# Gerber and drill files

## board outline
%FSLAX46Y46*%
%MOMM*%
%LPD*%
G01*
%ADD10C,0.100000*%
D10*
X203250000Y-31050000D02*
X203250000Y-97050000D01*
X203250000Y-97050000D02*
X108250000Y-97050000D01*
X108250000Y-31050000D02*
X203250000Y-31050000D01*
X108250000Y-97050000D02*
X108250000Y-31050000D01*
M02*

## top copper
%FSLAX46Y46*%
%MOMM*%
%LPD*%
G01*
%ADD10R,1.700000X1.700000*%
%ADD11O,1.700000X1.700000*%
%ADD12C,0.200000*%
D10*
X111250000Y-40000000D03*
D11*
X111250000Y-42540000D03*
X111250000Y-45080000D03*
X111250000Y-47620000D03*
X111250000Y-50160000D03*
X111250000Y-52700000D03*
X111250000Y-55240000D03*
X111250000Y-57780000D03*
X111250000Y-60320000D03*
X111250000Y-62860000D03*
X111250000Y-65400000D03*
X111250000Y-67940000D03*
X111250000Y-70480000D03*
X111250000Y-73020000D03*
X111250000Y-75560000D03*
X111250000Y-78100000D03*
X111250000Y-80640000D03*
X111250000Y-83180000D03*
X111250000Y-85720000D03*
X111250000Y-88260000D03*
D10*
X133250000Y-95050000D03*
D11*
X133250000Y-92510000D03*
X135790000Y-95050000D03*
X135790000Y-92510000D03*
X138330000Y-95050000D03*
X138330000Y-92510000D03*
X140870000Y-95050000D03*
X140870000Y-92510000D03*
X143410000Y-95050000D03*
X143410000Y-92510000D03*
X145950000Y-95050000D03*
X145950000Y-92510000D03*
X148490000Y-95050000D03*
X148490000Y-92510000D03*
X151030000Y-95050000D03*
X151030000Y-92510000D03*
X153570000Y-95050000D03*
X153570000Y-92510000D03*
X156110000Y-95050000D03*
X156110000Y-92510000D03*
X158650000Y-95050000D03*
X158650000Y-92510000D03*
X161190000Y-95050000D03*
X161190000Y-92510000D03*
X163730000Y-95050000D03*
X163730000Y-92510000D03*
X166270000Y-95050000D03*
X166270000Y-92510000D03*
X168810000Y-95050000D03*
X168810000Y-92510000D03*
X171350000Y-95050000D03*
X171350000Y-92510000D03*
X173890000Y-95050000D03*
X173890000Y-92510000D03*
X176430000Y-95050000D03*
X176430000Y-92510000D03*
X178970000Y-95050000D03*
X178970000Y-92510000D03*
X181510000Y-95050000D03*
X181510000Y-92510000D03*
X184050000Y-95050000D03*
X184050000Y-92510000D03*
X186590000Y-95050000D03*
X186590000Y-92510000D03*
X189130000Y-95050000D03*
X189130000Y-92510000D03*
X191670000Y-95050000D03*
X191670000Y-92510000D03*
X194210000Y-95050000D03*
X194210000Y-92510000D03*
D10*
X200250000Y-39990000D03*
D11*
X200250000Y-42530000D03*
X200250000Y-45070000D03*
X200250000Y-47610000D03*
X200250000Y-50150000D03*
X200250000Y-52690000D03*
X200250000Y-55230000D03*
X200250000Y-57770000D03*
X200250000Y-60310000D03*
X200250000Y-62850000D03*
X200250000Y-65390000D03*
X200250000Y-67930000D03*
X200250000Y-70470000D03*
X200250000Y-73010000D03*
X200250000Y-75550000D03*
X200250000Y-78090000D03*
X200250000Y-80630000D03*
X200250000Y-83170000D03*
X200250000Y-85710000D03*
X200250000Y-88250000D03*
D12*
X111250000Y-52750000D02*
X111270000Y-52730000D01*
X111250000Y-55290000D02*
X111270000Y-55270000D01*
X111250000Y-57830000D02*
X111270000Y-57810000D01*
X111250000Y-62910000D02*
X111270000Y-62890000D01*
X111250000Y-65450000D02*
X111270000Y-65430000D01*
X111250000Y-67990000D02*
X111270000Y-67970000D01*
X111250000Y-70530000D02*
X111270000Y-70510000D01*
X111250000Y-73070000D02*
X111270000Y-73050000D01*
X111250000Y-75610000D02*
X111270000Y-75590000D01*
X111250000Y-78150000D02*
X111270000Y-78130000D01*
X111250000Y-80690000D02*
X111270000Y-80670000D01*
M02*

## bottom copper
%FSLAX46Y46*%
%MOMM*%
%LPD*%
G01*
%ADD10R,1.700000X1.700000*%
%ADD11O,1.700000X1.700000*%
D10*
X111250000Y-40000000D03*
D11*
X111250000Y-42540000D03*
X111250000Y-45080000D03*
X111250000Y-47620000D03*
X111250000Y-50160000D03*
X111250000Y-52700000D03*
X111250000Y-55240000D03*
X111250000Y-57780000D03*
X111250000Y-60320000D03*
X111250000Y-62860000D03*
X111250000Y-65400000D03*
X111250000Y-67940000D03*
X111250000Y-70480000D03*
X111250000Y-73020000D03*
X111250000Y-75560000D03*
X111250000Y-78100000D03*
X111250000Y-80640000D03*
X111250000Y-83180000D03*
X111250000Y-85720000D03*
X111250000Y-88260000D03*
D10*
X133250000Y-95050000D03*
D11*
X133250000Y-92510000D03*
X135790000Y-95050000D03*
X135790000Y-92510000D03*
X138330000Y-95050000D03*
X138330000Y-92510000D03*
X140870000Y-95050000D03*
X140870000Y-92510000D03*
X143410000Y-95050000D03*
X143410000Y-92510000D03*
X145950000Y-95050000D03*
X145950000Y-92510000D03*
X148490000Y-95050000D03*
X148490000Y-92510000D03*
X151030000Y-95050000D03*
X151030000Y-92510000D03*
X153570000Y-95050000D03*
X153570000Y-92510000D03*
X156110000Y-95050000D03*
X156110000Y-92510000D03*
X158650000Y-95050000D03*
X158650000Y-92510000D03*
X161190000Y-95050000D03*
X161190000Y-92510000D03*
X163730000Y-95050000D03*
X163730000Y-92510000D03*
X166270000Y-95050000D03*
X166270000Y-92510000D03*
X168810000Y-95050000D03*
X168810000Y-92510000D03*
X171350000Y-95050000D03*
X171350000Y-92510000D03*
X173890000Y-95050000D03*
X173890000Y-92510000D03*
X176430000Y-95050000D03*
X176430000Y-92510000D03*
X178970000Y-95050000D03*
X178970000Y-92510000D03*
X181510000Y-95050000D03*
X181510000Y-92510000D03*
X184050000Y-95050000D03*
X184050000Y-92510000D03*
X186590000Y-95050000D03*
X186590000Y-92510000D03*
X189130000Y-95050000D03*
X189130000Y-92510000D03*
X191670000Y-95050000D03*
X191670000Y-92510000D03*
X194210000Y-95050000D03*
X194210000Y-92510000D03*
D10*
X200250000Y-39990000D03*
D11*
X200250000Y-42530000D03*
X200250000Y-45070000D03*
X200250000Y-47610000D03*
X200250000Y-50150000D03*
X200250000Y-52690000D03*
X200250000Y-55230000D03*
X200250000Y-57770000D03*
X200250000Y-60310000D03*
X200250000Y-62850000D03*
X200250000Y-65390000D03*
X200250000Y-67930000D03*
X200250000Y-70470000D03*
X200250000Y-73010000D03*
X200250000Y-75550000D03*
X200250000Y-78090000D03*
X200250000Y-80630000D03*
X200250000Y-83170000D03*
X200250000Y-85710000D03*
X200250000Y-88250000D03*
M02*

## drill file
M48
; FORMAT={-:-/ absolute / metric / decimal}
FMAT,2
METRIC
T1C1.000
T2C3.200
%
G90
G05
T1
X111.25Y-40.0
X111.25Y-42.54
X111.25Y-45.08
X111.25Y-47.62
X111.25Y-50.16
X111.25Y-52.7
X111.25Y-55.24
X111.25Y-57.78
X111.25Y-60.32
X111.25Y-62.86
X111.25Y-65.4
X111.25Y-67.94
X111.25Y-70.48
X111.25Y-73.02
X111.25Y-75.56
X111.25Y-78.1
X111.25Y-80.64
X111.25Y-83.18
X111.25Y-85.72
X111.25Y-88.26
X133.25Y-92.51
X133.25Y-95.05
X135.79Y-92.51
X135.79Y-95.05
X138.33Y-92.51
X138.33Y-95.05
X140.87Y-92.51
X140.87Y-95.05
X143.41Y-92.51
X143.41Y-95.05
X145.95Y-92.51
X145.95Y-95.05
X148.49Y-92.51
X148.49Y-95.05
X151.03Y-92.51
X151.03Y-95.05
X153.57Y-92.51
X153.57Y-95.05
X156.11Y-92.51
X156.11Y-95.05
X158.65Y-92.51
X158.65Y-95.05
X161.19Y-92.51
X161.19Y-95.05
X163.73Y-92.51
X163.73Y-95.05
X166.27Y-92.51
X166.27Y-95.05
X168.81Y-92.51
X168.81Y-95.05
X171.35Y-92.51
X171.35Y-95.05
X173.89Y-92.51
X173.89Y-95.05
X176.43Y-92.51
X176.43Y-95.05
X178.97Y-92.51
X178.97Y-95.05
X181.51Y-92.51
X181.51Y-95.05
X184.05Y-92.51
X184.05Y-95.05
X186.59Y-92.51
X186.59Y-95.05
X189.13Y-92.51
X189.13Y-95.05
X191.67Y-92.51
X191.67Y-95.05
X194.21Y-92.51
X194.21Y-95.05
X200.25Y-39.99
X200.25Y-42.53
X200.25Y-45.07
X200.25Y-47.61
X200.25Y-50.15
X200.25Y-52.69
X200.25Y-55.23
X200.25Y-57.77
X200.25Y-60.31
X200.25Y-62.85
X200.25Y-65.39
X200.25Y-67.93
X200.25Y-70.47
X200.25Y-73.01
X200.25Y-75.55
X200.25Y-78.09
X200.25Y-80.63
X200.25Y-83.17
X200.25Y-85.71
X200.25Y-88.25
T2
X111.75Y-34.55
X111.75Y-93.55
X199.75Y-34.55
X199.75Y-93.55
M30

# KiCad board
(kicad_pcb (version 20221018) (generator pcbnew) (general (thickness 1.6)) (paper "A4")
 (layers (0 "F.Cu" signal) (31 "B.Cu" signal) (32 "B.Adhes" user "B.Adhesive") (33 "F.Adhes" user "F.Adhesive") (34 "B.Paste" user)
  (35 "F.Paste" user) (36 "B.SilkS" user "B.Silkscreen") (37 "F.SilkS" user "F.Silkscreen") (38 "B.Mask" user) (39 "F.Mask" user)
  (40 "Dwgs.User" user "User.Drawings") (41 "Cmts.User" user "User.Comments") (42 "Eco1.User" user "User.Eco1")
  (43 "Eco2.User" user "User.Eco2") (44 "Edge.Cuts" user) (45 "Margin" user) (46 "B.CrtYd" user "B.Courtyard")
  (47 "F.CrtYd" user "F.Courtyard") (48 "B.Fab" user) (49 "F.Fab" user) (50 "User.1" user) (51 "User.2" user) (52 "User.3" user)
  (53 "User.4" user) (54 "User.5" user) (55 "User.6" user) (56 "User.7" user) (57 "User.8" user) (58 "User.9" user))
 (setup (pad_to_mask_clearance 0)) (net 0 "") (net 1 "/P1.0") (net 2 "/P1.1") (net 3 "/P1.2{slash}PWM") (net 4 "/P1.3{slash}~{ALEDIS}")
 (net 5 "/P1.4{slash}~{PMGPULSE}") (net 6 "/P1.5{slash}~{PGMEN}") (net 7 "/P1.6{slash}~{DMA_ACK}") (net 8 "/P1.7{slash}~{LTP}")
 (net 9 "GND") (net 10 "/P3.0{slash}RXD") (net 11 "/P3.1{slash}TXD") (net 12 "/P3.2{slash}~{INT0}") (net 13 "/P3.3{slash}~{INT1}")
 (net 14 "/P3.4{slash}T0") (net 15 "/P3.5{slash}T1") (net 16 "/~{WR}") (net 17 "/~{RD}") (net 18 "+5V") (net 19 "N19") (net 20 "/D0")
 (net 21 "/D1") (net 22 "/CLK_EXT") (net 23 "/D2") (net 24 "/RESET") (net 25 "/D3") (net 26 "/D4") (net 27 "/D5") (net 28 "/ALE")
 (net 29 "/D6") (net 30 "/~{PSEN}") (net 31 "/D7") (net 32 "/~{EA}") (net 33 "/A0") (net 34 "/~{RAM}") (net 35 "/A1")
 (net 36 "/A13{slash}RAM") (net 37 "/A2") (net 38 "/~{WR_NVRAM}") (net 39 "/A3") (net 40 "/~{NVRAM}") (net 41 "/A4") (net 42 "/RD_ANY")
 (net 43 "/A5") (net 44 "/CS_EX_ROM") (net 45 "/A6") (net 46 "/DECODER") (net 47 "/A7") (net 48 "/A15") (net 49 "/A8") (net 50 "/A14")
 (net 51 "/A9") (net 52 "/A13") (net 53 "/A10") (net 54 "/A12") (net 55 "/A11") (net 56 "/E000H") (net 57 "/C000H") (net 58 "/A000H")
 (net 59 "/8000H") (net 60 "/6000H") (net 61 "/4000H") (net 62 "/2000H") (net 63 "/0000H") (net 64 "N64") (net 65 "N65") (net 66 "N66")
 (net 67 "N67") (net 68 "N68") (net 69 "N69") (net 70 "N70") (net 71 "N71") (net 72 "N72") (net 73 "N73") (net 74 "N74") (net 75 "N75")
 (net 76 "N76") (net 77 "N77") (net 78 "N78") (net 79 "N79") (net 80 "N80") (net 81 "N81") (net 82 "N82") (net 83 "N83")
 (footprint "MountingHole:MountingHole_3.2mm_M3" (layer "F.Cu") (at 199.75 93.55)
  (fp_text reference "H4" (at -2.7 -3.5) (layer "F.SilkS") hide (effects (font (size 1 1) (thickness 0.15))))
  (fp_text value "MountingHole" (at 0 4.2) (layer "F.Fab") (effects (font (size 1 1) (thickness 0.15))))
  (pad "" np_thru_hole circle (at 0 0) (size 3.2 3.2) (drill 3.2) (layers "F&B.Cu" "*.Mask")))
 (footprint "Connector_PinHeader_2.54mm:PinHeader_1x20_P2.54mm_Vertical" (layer "F.Cu") (at 111.25 40)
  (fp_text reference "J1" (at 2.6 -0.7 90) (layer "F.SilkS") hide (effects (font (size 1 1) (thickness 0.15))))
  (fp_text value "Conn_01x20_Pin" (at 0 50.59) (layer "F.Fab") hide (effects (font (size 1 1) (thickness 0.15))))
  (pad "1" thru_hole rect (at 0 0) (size 1.7 1.7) (drill 1) (layers "*.Cu" "*.Mask") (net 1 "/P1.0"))
  (pad "2" thru_hole oval (at 0 2.54) (size 1.7 1.7) (drill 1) (layers "*.Cu" "*.Mask") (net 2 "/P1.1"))
  (pad "3" thru_hole oval (at 0 5.08) (size 1.7 1.7) (drill 1) (layers "*.Cu" "*.Mask") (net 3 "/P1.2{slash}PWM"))
  (pad "4" thru_hole oval (at 0 7.62) (size 1.7 1.7) (drill 1) (layers "*.Cu" "*.Mask") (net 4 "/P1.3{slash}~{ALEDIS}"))
  (pad "5" thru_hole oval (at 0 10.16) (size 1.7 1.7) (drill 1) (layers "*.Cu" "*.Mask") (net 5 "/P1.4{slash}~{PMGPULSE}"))
  (pad "6" thru_hole oval (at 0 12.7) (size 1.7 1.7) (drill 1) (layers "*.Cu" "*.Mask") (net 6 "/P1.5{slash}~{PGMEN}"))
  (pad "7" thru_hole oval (at 0 15.24) (size 1.7 1.7) (drill 1) (layers "*.Cu" "*.Mask") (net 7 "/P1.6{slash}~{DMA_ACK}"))
  (pad "8" thru_hole oval (at 0 17.78) (size 1.7 1.7) (drill 1) (layers "*.Cu" "*.Mask") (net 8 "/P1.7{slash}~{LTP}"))
  (pad "9" thru_hole oval (at 0 20.32) (size 1.7 1.7) (drill 1) (layers "*.Cu" "*.Mask") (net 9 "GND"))
  (pad "10" thru_hole oval (at 0 22.86) (size 1.7 1.7) (drill 1) (layers "*.Cu" "*.Mask") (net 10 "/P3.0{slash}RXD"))
  (pad "11" thru_hole oval (at 0 25.4) (size 1.7 1.7) (drill 1) (layers "*.Cu" "*.Mask") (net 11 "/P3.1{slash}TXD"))
  (pad "12" thru_hole oval (at 0 27.94) (size 1.7 1.7) (drill 1) (layers "*.Cu" "*.Mask") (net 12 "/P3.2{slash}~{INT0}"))
  (pad "13" thru_hole oval (at 0 30.48) (size 1.7 1.7) (drill 1) (layers "*.Cu" "*.Mask") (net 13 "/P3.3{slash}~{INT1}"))
  (pad "14" thru_hole oval (at 0 33.02) (size 1.7 1.7) (drill 1) (layers "*.Cu" "*.Mask") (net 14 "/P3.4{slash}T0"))
  (pad "15" thru_hole oval (at 0 35.56) (size 1.7 1.7) (drill 1) (layers "*.Cu" "*.Mask") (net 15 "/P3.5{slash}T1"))
  (pad "16" thru_hole oval (at 0 38.1) (size 1.7 1.7) (drill 1) (layers "*.Cu" "*.Mask") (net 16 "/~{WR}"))
  (pad "17" thru_hole oval (at 0 40.64) (size 1.7 1.7) (drill 1) (layers "*.Cu" "*.Mask") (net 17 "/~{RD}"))
  (pad "18" thru_hole oval (at 0 43.18) (size 1.7 1.7) (drill 1) (layers "*.Cu" "*.Mask") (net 9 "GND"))
  (pad "19" thru_hole oval (at 0 45.72) (size 1.7 1.7) (drill 1) (layers "*.Cu" "*.Mask") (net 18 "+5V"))
  (pad "20" thru_hole oval (at 0 48.26) (size 1.7 1.7) (drill 1) (layers "*.Cu" "*.Mask") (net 18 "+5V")))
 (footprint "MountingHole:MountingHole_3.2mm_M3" (layer "F.Cu") (at 111.75 34.55)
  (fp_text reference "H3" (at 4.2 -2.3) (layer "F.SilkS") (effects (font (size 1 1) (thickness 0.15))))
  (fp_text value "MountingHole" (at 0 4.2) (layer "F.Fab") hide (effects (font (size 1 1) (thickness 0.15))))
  (pad "" np_thru_hole circle (at 0 0) (size 3.2 3.2) (drill 3.2) (layers "F&B.Cu" "*.Mask")))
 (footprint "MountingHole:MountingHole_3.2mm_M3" (layer "F.Cu") (at 111.75 93.55)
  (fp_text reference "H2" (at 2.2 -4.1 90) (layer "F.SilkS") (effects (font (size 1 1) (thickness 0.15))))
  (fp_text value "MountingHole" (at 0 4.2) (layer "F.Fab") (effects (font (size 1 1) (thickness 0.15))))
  (pad "" np_thru_hole circle (at 0 0) (size 3.2 3.2) (drill 3.2) (layers "F&B.Cu" "*.Mask")))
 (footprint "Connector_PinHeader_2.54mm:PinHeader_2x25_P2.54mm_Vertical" (layer "F.Cu") (at 133.25 95.05 90)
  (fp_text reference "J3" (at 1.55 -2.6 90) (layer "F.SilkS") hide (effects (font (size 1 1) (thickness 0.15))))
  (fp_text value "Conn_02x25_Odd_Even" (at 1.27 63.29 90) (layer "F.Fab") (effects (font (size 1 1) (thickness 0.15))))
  (pad "1" thru_hole rect (at 0 0 90) (size 1.7 1.7) (drill 1) (layers "*.Cu" "*.Mask") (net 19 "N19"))
  (pad "2" thru_hole oval (at 2.54 0 90) (size 1.7 1.7) (drill 1) (layers "*.Cu" "*.Mask") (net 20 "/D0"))
  (pad "3" thru_hole oval (at 0 2.54 90) (size 1.7 1.7) (drill 1) (layers "*.Cu" "*.Mask") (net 9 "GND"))
  (pad "4" thru_hole oval (at 2.54 2.54 90) (size 1.7 1.7) (drill 1) (layers "*.Cu" "*.Mask") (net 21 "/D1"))
  (pad "5" thru_hole oval (at 0 5.08 90) (size 1.7 1.7) (drill 1) (layers "*.Cu" "*.Mask") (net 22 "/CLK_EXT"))
  (pad "6" thru_hole oval (at 2.54 5.08 90) (size 1.7 1.7) (drill 1) (layers "*.Cu" "*.Mask") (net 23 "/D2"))
  (pad "7" thru_hole oval (at 0 7.62 90) (size 1.7 1.7) (drill 1) (layers "*.Cu" "*.Mask") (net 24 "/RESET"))
  (pad "8" thru_hole oval (at 2.54 7.62 90) (size 1.7 1.7) (drill 1) (layers "*.Cu" "*.Mask") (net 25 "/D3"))
  (pad "9" thru_hole oval (at 0 10.16 90) (size 1.7 1.7) (drill 1) (layers "*.Cu" "*.Mask") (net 16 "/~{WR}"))
  (pad "10" thru_hole oval (at 2.54 10.16 90) (size 1.7 1.7) (drill 1) (layers "*.Cu" "*.Mask") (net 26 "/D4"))
  (pad "11" thru_hole oval (at 0 12.7 90) (size 1.7 1.7) (drill 1) (layers "*.Cu" "*.Mask") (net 17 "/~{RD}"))
  (pad "12" thru_hole oval (at 2.54 12.7 90) (size 1.7 1.7) (drill 1) (layers "*.Cu" "*.Mask") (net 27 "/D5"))
  (pad "13" thru_hole oval (at 0 15.24 90) (size 1.7 1.7) (drill 1) (layers "*.Cu" "*.Mask") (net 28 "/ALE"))
  (pad "14" thru_hole oval (at 2.54 15.24 90) (size 1.7 1.7) (drill 1) (layers "*.Cu" "*.Mask") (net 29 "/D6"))
  (pad "15" thru_hole oval (at 0 17.78 90) (size 1.7 1.7) (drill 1) (layers "*.Cu" "*.Mask") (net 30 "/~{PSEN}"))
  (pad "16" thru_hole oval (at 2.54 17.78 90) (size 1.7 1.7) (drill 1) (layers "*.Cu" "*.Mask") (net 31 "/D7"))
  (pad "17" thru_hole oval (at 0 20.32 90) (size 1.7 1.7) (drill 1) (layers "*.Cu" "*.Mask") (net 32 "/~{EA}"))
  (pad "18" thru_hole oval (at 2.54 20.32 90) (size 1.7 1.7) (drill 1) (layers "*.Cu" "*.Mask") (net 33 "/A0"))
  (pad "19" thru_hole oval (at 0 22.86 90) (size 1.7 1.7) (drill 1) (layers "*.Cu" "*.Mask") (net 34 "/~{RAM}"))
  (pad "20" thru_hole oval (at 2.54 22.86 90) (size 1.7 1.7) (drill 1) (layers "*.Cu" "*.Mask") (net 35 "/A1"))
  (pad "21" thru_hole oval (at 0 25.4 90) (size 1.7 1.7) (drill 1) (layers "*.Cu" "*.Mask") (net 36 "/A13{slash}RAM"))
  (pad "22" thru_hole oval (at 2.54 25.4 90) (size 1.7 1.7) (drill 1) (layers "*.Cu" "*.Mask") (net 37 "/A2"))
  (pad "23" thru_hole oval (at 0 27.94 90) (size 1.7 1.7) (drill 1) (layers "*.Cu" "*.Mask") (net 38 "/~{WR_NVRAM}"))
  (pad "24" thru_hole oval (at 2.54 27.94 90) (size 1.7 1.7) (drill 1) (layers "*.Cu" "*.Mask") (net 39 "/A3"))
  (pad "25" thru_hole oval (at 0 30.48 90) (size 1.7 1.7) (drill 1) (layers "*.Cu" "*.Mask") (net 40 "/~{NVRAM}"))
  (pad "26" thru_hole oval (at 2.54 30.48 90) (size 1.7 1.7) (drill 1) (layers "*.Cu" "*.Mask") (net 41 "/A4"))
  (pad "27" thru_hole oval (at 0 33.02 90) (size 1.7 1.7) (drill 1) (layers "*.Cu" "*.Mask") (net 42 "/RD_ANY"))
  (pad "28" thru_hole oval (at 2.54 33.02 90) (size 1.7 1.7) (drill 1) (layers "*.Cu" "*.Mask") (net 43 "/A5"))
  (pad "29" thru_hole oval (at 0 35.56 90) (size 1.7 1.7) (drill 1) (layers "*.Cu" "*.Mask") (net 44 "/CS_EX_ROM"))
  (pad "30" thru_hole oval (at 2.54 35.56 90) (size 1.7 1.7) (drill 1) (layers "*.Cu" "*.Mask") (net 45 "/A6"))
  (pad "31" thru_hole oval (at 0 38.1 90) (size 1.7 1.7) (drill 1) (layers "*.Cu" "*.Mask") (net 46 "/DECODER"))
  (pad "32" thru_hole oval (at 2.54 38.1 90) (size 1.7 1.7) (drill 1) (layers "*.Cu" "*.Mask") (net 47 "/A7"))
  (pad "33" thru_hole oval (at 0 40.64 90) (size 1.7 1.7) (drill 1) (layers "*.Cu" "*.Mask") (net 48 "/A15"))
  (pad "34" thru_hole oval (at 2.54 40.64 90) (size 1.7 1.7) (drill 1) (layers "*.Cu" "*.Mask") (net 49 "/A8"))
  (pad "35" thru_hole oval (at 0 43.18 90) (size 1.7 1.7) (drill 1) (layers "*.Cu" "*.Mask") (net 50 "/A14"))
  (pad "36" thru_hole oval (at 2.54 43.18 90) (size 1.7 1.7) (drill 1) (layers "*.Cu" "*.Mask") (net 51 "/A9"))
  (pad "37" thru_hole oval (at 0 45.72 90) (size 1.7 1.7) (drill 1) (layers "*.Cu" "*.Mask") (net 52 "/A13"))
  (pad "38" thru_hole oval (at 2.54 45.72 90) (size 1.7 1.7) (drill 1) (layers "*.Cu" "*.Mask") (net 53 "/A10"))
  (pad "39" thru_hole oval (at 0 48.26 90) (size 1.7 1.7) (drill 1) (layers "*.Cu" "*.Mask") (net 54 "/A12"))
  (pad "40" thru_hole oval (at 2.54 48.26 90) (size 1.7 1.7) (drill 1) (layers "*.Cu" "*.Mask") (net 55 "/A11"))
  (pad "41" thru_hole oval (at 0 50.8 90) (size 1.7 1.7) (drill 1) (layers "*.Cu" "*.Mask") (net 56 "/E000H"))
  (pad "42" thru_hole oval (at 2.54 50.8 90) (size 1.7 1.7) (drill 1) (layers "*.Cu" "*.Mask") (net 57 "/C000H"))
  (pad "43" thru_hole oval (at 0 53.34 90) (size 1.7 1.7) (drill 1) (layers "*.Cu" "*.Mask") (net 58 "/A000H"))
  (pad "44" thru_hole oval (at 2.54 53.34 90) (size 1.7 1.7) (drill 1) (layers "*.Cu" "*.Mask") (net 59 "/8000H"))
  (pad "45" thru_hole oval (at 0 55.88 90) (size 1.7 1.7) (drill 1) (layers "*.Cu" "*.Mask") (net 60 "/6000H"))
  (pad "46" thru_hole oval (at 2.54 55.88 90) (size 1.7 1.7) (drill 1) (layers "*.Cu" "*.Mask") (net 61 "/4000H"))
  (pad "47" thru_hole oval (at 0 58.42 90) (size 1.7 1.7) (drill 1) (layers "*.Cu" "*.Mask") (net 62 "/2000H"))
  (pad "48" thru_hole oval (at 2.54 58.42 90) (size 1.7 1.7) (drill 1) (layers "*.Cu" "*.Mask") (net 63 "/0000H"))
  (pad "49" thru_hole oval (at 0 60.96 90) (size 1.7 1.7) (drill 1) (layers "*.Cu" "*.Mask") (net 9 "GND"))
  (pad "50" thru_hole oval (at 2.54 60.96 90) (size 1.7 1.7) (drill 1) (layers "*.Cu" "*.Mask") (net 18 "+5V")))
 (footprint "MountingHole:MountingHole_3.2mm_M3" (layer "F.Cu") (at 199.75 34.55)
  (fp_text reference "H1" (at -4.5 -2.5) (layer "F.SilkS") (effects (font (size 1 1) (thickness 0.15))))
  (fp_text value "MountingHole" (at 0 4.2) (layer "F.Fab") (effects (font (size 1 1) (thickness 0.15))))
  (pad "" np_thru_hole circle (at 0 0) (size 3.2 3.2) (drill 3.2) (layers "F&B.Cu" "*.Mask")))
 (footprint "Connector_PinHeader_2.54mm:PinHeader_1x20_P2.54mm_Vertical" (layer "F.Cu") (at 200.25 39.99)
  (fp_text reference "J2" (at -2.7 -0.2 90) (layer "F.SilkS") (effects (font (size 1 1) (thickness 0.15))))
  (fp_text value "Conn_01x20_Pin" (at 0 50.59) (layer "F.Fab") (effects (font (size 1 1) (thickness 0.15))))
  (pad "1" thru_hole rect (at 0 0) (size 1.7 1.7) (drill 1) (layers "*.Cu" "*.Mask") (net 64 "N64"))
  (pad "2" thru_hole oval (at 0 2.54) (size 1.7 1.7) (drill 1) (layers "*.Cu" "*.Mask") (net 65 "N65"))
  (pad "3" thru_hole oval (at 0 5.08) (size 1.7 1.7) (drill 1) (layers "*.Cu" "*.Mask") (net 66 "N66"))
  (pad "4" thru_hole oval (at 0 7.62) (size 1.7 1.7) (drill 1) (layers "*.Cu" "*.Mask") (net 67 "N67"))
  (pad "5" thru_hole oval (at 0 10.16) (size 1.7 1.7) (drill 1) (layers "*.Cu" "*.Mask") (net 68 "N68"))
  (pad "6" thru_hole oval (at 0 12.7) (size 1.7 1.7) (drill 1) (layers "*.Cu" "*.Mask") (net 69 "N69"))
  (pad "7" thru_hole oval (at 0 15.24) (size 1.7 1.7) (drill 1) (layers "*.Cu" "*.Mask") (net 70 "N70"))
  (pad "8" thru_hole oval (at 0 17.78) (size 1.7 1.7) (drill 1) (layers "*.Cu" "*.Mask") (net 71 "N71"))
  (pad "9" thru_hole oval (at 0 20.32) (size 1.7 1.7) (drill 1) (layers "*.Cu" "*.Mask") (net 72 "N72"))
  (pad "10" thru_hole oval (at 0 22.86) (size 1.7 1.7) (drill 1) (layers "*.Cu" "*.Mask") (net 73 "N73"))
  (pad "11" thru_hole oval (at 0 25.4) (size 1.7 1.7) (drill 1) (layers "*.Cu" "*.Mask") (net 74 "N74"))
  (pad "12" thru_hole oval (at 0 27.94) (size 1.7 1.7) (drill 1) (layers "*.Cu" "*.Mask") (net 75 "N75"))
  (pad "13" thru_hole oval (at 0 30.48) (size 1.7 1.7) (drill 1) (layers "*.Cu" "*.Mask") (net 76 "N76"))
  (pad "14" thru_hole oval (at 0 33.02) (size 1.7 1.7) (drill 1) (layers "*.Cu" "*.Mask") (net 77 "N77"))
  (pad "15" thru_hole oval (at 0 35.56) (size 1.7 1.7) (drill 1) (layers "*.Cu" "*.Mask") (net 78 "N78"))
  (pad "16" thru_hole oval (at 0 38.1) (size 1.7 1.7) (drill 1) (layers "*.Cu" "*.Mask") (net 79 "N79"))
  (pad "17" thru_hole oval (at 0 40.64) (size 1.7 1.7) (drill 1) (layers "*.Cu" "*.Mask") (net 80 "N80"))
  (pad "18" thru_hole oval (at 0 43.18) (size 1.7 1.7) (drill 1) (layers "*.Cu" "*.Mask") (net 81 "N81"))
  (pad "19" thru_hole oval (at 0 45.72) (size 1.7 1.7) (drill 1) (layers "*.Cu" "*.Mask") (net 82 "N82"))
  (pad "20" thru_hole oval (at 0 48.26) (size 1.7 1.7) (drill 1) (layers "*.Cu" "*.Mask") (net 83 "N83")))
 (gr_line (start 203.25 31.05) (end 203.25 97.05) (stroke (width 0.1) (type solid)) (layer "Edge.Cuts"))
 (gr_line (start 203.25 97.05) (end 108.25 97.05) (stroke (width 0.1) (type solid)) (layer "Edge.Cuts"))
 (gr_line (start 108.25 31.05) (end 203.25 31.05) (stroke (width 0.1) (type solid)) (layer "Edge.Cuts"))
 (gr_line (start 108.25 97.05) (end 108.25 31.05) (stroke (width 0.1) (type solid)) (layer "Edge.Cuts"))
 (segment (start 111.25 52.75) (end 111.27 52.73) (width 0.2) (layer "F.Cu") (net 6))
 (segment (start 111.25 55.29) (end 111.27 55.27) (width 0.2) (layer "F.Cu") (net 7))
 (segment (start 111.25 57.83) (end 111.27 57.81) (width 0.2) (layer "F.Cu") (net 8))
 (segment (start 111.25 62.91) (end 111.27 62.89) (width 0.2) (layer "F.Cu") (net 10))
 (segment (start 111.25 65.45) (end 111.27 65.43) (width 0.2) (layer "F.Cu") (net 11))
 (segment (start 111.25 67.99) (end 111.27 67.97) (width 0.2) (layer "F.Cu") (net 12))
 (segment (start 111.25 70.53) (end 111.27 70.51) (width 0.2) (layer "F.Cu") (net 13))
 (segment (start 111.25 73.07) (end 111.27 73.05) (width 0.2) (layer "F.Cu") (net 14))
 (segment (start 111.25 75.61) (end 111.27 75.59) (width 0.2) (layer "F.Cu") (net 15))
 (segment (start 111.25 78.15) (end 111.27 78.13) (width 0.2) (layer "F.Cu") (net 16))
 (segment (start 111.25 80.69) (end 111.27 80.67) (width 0.2) (layer "F.Cu") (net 17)))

